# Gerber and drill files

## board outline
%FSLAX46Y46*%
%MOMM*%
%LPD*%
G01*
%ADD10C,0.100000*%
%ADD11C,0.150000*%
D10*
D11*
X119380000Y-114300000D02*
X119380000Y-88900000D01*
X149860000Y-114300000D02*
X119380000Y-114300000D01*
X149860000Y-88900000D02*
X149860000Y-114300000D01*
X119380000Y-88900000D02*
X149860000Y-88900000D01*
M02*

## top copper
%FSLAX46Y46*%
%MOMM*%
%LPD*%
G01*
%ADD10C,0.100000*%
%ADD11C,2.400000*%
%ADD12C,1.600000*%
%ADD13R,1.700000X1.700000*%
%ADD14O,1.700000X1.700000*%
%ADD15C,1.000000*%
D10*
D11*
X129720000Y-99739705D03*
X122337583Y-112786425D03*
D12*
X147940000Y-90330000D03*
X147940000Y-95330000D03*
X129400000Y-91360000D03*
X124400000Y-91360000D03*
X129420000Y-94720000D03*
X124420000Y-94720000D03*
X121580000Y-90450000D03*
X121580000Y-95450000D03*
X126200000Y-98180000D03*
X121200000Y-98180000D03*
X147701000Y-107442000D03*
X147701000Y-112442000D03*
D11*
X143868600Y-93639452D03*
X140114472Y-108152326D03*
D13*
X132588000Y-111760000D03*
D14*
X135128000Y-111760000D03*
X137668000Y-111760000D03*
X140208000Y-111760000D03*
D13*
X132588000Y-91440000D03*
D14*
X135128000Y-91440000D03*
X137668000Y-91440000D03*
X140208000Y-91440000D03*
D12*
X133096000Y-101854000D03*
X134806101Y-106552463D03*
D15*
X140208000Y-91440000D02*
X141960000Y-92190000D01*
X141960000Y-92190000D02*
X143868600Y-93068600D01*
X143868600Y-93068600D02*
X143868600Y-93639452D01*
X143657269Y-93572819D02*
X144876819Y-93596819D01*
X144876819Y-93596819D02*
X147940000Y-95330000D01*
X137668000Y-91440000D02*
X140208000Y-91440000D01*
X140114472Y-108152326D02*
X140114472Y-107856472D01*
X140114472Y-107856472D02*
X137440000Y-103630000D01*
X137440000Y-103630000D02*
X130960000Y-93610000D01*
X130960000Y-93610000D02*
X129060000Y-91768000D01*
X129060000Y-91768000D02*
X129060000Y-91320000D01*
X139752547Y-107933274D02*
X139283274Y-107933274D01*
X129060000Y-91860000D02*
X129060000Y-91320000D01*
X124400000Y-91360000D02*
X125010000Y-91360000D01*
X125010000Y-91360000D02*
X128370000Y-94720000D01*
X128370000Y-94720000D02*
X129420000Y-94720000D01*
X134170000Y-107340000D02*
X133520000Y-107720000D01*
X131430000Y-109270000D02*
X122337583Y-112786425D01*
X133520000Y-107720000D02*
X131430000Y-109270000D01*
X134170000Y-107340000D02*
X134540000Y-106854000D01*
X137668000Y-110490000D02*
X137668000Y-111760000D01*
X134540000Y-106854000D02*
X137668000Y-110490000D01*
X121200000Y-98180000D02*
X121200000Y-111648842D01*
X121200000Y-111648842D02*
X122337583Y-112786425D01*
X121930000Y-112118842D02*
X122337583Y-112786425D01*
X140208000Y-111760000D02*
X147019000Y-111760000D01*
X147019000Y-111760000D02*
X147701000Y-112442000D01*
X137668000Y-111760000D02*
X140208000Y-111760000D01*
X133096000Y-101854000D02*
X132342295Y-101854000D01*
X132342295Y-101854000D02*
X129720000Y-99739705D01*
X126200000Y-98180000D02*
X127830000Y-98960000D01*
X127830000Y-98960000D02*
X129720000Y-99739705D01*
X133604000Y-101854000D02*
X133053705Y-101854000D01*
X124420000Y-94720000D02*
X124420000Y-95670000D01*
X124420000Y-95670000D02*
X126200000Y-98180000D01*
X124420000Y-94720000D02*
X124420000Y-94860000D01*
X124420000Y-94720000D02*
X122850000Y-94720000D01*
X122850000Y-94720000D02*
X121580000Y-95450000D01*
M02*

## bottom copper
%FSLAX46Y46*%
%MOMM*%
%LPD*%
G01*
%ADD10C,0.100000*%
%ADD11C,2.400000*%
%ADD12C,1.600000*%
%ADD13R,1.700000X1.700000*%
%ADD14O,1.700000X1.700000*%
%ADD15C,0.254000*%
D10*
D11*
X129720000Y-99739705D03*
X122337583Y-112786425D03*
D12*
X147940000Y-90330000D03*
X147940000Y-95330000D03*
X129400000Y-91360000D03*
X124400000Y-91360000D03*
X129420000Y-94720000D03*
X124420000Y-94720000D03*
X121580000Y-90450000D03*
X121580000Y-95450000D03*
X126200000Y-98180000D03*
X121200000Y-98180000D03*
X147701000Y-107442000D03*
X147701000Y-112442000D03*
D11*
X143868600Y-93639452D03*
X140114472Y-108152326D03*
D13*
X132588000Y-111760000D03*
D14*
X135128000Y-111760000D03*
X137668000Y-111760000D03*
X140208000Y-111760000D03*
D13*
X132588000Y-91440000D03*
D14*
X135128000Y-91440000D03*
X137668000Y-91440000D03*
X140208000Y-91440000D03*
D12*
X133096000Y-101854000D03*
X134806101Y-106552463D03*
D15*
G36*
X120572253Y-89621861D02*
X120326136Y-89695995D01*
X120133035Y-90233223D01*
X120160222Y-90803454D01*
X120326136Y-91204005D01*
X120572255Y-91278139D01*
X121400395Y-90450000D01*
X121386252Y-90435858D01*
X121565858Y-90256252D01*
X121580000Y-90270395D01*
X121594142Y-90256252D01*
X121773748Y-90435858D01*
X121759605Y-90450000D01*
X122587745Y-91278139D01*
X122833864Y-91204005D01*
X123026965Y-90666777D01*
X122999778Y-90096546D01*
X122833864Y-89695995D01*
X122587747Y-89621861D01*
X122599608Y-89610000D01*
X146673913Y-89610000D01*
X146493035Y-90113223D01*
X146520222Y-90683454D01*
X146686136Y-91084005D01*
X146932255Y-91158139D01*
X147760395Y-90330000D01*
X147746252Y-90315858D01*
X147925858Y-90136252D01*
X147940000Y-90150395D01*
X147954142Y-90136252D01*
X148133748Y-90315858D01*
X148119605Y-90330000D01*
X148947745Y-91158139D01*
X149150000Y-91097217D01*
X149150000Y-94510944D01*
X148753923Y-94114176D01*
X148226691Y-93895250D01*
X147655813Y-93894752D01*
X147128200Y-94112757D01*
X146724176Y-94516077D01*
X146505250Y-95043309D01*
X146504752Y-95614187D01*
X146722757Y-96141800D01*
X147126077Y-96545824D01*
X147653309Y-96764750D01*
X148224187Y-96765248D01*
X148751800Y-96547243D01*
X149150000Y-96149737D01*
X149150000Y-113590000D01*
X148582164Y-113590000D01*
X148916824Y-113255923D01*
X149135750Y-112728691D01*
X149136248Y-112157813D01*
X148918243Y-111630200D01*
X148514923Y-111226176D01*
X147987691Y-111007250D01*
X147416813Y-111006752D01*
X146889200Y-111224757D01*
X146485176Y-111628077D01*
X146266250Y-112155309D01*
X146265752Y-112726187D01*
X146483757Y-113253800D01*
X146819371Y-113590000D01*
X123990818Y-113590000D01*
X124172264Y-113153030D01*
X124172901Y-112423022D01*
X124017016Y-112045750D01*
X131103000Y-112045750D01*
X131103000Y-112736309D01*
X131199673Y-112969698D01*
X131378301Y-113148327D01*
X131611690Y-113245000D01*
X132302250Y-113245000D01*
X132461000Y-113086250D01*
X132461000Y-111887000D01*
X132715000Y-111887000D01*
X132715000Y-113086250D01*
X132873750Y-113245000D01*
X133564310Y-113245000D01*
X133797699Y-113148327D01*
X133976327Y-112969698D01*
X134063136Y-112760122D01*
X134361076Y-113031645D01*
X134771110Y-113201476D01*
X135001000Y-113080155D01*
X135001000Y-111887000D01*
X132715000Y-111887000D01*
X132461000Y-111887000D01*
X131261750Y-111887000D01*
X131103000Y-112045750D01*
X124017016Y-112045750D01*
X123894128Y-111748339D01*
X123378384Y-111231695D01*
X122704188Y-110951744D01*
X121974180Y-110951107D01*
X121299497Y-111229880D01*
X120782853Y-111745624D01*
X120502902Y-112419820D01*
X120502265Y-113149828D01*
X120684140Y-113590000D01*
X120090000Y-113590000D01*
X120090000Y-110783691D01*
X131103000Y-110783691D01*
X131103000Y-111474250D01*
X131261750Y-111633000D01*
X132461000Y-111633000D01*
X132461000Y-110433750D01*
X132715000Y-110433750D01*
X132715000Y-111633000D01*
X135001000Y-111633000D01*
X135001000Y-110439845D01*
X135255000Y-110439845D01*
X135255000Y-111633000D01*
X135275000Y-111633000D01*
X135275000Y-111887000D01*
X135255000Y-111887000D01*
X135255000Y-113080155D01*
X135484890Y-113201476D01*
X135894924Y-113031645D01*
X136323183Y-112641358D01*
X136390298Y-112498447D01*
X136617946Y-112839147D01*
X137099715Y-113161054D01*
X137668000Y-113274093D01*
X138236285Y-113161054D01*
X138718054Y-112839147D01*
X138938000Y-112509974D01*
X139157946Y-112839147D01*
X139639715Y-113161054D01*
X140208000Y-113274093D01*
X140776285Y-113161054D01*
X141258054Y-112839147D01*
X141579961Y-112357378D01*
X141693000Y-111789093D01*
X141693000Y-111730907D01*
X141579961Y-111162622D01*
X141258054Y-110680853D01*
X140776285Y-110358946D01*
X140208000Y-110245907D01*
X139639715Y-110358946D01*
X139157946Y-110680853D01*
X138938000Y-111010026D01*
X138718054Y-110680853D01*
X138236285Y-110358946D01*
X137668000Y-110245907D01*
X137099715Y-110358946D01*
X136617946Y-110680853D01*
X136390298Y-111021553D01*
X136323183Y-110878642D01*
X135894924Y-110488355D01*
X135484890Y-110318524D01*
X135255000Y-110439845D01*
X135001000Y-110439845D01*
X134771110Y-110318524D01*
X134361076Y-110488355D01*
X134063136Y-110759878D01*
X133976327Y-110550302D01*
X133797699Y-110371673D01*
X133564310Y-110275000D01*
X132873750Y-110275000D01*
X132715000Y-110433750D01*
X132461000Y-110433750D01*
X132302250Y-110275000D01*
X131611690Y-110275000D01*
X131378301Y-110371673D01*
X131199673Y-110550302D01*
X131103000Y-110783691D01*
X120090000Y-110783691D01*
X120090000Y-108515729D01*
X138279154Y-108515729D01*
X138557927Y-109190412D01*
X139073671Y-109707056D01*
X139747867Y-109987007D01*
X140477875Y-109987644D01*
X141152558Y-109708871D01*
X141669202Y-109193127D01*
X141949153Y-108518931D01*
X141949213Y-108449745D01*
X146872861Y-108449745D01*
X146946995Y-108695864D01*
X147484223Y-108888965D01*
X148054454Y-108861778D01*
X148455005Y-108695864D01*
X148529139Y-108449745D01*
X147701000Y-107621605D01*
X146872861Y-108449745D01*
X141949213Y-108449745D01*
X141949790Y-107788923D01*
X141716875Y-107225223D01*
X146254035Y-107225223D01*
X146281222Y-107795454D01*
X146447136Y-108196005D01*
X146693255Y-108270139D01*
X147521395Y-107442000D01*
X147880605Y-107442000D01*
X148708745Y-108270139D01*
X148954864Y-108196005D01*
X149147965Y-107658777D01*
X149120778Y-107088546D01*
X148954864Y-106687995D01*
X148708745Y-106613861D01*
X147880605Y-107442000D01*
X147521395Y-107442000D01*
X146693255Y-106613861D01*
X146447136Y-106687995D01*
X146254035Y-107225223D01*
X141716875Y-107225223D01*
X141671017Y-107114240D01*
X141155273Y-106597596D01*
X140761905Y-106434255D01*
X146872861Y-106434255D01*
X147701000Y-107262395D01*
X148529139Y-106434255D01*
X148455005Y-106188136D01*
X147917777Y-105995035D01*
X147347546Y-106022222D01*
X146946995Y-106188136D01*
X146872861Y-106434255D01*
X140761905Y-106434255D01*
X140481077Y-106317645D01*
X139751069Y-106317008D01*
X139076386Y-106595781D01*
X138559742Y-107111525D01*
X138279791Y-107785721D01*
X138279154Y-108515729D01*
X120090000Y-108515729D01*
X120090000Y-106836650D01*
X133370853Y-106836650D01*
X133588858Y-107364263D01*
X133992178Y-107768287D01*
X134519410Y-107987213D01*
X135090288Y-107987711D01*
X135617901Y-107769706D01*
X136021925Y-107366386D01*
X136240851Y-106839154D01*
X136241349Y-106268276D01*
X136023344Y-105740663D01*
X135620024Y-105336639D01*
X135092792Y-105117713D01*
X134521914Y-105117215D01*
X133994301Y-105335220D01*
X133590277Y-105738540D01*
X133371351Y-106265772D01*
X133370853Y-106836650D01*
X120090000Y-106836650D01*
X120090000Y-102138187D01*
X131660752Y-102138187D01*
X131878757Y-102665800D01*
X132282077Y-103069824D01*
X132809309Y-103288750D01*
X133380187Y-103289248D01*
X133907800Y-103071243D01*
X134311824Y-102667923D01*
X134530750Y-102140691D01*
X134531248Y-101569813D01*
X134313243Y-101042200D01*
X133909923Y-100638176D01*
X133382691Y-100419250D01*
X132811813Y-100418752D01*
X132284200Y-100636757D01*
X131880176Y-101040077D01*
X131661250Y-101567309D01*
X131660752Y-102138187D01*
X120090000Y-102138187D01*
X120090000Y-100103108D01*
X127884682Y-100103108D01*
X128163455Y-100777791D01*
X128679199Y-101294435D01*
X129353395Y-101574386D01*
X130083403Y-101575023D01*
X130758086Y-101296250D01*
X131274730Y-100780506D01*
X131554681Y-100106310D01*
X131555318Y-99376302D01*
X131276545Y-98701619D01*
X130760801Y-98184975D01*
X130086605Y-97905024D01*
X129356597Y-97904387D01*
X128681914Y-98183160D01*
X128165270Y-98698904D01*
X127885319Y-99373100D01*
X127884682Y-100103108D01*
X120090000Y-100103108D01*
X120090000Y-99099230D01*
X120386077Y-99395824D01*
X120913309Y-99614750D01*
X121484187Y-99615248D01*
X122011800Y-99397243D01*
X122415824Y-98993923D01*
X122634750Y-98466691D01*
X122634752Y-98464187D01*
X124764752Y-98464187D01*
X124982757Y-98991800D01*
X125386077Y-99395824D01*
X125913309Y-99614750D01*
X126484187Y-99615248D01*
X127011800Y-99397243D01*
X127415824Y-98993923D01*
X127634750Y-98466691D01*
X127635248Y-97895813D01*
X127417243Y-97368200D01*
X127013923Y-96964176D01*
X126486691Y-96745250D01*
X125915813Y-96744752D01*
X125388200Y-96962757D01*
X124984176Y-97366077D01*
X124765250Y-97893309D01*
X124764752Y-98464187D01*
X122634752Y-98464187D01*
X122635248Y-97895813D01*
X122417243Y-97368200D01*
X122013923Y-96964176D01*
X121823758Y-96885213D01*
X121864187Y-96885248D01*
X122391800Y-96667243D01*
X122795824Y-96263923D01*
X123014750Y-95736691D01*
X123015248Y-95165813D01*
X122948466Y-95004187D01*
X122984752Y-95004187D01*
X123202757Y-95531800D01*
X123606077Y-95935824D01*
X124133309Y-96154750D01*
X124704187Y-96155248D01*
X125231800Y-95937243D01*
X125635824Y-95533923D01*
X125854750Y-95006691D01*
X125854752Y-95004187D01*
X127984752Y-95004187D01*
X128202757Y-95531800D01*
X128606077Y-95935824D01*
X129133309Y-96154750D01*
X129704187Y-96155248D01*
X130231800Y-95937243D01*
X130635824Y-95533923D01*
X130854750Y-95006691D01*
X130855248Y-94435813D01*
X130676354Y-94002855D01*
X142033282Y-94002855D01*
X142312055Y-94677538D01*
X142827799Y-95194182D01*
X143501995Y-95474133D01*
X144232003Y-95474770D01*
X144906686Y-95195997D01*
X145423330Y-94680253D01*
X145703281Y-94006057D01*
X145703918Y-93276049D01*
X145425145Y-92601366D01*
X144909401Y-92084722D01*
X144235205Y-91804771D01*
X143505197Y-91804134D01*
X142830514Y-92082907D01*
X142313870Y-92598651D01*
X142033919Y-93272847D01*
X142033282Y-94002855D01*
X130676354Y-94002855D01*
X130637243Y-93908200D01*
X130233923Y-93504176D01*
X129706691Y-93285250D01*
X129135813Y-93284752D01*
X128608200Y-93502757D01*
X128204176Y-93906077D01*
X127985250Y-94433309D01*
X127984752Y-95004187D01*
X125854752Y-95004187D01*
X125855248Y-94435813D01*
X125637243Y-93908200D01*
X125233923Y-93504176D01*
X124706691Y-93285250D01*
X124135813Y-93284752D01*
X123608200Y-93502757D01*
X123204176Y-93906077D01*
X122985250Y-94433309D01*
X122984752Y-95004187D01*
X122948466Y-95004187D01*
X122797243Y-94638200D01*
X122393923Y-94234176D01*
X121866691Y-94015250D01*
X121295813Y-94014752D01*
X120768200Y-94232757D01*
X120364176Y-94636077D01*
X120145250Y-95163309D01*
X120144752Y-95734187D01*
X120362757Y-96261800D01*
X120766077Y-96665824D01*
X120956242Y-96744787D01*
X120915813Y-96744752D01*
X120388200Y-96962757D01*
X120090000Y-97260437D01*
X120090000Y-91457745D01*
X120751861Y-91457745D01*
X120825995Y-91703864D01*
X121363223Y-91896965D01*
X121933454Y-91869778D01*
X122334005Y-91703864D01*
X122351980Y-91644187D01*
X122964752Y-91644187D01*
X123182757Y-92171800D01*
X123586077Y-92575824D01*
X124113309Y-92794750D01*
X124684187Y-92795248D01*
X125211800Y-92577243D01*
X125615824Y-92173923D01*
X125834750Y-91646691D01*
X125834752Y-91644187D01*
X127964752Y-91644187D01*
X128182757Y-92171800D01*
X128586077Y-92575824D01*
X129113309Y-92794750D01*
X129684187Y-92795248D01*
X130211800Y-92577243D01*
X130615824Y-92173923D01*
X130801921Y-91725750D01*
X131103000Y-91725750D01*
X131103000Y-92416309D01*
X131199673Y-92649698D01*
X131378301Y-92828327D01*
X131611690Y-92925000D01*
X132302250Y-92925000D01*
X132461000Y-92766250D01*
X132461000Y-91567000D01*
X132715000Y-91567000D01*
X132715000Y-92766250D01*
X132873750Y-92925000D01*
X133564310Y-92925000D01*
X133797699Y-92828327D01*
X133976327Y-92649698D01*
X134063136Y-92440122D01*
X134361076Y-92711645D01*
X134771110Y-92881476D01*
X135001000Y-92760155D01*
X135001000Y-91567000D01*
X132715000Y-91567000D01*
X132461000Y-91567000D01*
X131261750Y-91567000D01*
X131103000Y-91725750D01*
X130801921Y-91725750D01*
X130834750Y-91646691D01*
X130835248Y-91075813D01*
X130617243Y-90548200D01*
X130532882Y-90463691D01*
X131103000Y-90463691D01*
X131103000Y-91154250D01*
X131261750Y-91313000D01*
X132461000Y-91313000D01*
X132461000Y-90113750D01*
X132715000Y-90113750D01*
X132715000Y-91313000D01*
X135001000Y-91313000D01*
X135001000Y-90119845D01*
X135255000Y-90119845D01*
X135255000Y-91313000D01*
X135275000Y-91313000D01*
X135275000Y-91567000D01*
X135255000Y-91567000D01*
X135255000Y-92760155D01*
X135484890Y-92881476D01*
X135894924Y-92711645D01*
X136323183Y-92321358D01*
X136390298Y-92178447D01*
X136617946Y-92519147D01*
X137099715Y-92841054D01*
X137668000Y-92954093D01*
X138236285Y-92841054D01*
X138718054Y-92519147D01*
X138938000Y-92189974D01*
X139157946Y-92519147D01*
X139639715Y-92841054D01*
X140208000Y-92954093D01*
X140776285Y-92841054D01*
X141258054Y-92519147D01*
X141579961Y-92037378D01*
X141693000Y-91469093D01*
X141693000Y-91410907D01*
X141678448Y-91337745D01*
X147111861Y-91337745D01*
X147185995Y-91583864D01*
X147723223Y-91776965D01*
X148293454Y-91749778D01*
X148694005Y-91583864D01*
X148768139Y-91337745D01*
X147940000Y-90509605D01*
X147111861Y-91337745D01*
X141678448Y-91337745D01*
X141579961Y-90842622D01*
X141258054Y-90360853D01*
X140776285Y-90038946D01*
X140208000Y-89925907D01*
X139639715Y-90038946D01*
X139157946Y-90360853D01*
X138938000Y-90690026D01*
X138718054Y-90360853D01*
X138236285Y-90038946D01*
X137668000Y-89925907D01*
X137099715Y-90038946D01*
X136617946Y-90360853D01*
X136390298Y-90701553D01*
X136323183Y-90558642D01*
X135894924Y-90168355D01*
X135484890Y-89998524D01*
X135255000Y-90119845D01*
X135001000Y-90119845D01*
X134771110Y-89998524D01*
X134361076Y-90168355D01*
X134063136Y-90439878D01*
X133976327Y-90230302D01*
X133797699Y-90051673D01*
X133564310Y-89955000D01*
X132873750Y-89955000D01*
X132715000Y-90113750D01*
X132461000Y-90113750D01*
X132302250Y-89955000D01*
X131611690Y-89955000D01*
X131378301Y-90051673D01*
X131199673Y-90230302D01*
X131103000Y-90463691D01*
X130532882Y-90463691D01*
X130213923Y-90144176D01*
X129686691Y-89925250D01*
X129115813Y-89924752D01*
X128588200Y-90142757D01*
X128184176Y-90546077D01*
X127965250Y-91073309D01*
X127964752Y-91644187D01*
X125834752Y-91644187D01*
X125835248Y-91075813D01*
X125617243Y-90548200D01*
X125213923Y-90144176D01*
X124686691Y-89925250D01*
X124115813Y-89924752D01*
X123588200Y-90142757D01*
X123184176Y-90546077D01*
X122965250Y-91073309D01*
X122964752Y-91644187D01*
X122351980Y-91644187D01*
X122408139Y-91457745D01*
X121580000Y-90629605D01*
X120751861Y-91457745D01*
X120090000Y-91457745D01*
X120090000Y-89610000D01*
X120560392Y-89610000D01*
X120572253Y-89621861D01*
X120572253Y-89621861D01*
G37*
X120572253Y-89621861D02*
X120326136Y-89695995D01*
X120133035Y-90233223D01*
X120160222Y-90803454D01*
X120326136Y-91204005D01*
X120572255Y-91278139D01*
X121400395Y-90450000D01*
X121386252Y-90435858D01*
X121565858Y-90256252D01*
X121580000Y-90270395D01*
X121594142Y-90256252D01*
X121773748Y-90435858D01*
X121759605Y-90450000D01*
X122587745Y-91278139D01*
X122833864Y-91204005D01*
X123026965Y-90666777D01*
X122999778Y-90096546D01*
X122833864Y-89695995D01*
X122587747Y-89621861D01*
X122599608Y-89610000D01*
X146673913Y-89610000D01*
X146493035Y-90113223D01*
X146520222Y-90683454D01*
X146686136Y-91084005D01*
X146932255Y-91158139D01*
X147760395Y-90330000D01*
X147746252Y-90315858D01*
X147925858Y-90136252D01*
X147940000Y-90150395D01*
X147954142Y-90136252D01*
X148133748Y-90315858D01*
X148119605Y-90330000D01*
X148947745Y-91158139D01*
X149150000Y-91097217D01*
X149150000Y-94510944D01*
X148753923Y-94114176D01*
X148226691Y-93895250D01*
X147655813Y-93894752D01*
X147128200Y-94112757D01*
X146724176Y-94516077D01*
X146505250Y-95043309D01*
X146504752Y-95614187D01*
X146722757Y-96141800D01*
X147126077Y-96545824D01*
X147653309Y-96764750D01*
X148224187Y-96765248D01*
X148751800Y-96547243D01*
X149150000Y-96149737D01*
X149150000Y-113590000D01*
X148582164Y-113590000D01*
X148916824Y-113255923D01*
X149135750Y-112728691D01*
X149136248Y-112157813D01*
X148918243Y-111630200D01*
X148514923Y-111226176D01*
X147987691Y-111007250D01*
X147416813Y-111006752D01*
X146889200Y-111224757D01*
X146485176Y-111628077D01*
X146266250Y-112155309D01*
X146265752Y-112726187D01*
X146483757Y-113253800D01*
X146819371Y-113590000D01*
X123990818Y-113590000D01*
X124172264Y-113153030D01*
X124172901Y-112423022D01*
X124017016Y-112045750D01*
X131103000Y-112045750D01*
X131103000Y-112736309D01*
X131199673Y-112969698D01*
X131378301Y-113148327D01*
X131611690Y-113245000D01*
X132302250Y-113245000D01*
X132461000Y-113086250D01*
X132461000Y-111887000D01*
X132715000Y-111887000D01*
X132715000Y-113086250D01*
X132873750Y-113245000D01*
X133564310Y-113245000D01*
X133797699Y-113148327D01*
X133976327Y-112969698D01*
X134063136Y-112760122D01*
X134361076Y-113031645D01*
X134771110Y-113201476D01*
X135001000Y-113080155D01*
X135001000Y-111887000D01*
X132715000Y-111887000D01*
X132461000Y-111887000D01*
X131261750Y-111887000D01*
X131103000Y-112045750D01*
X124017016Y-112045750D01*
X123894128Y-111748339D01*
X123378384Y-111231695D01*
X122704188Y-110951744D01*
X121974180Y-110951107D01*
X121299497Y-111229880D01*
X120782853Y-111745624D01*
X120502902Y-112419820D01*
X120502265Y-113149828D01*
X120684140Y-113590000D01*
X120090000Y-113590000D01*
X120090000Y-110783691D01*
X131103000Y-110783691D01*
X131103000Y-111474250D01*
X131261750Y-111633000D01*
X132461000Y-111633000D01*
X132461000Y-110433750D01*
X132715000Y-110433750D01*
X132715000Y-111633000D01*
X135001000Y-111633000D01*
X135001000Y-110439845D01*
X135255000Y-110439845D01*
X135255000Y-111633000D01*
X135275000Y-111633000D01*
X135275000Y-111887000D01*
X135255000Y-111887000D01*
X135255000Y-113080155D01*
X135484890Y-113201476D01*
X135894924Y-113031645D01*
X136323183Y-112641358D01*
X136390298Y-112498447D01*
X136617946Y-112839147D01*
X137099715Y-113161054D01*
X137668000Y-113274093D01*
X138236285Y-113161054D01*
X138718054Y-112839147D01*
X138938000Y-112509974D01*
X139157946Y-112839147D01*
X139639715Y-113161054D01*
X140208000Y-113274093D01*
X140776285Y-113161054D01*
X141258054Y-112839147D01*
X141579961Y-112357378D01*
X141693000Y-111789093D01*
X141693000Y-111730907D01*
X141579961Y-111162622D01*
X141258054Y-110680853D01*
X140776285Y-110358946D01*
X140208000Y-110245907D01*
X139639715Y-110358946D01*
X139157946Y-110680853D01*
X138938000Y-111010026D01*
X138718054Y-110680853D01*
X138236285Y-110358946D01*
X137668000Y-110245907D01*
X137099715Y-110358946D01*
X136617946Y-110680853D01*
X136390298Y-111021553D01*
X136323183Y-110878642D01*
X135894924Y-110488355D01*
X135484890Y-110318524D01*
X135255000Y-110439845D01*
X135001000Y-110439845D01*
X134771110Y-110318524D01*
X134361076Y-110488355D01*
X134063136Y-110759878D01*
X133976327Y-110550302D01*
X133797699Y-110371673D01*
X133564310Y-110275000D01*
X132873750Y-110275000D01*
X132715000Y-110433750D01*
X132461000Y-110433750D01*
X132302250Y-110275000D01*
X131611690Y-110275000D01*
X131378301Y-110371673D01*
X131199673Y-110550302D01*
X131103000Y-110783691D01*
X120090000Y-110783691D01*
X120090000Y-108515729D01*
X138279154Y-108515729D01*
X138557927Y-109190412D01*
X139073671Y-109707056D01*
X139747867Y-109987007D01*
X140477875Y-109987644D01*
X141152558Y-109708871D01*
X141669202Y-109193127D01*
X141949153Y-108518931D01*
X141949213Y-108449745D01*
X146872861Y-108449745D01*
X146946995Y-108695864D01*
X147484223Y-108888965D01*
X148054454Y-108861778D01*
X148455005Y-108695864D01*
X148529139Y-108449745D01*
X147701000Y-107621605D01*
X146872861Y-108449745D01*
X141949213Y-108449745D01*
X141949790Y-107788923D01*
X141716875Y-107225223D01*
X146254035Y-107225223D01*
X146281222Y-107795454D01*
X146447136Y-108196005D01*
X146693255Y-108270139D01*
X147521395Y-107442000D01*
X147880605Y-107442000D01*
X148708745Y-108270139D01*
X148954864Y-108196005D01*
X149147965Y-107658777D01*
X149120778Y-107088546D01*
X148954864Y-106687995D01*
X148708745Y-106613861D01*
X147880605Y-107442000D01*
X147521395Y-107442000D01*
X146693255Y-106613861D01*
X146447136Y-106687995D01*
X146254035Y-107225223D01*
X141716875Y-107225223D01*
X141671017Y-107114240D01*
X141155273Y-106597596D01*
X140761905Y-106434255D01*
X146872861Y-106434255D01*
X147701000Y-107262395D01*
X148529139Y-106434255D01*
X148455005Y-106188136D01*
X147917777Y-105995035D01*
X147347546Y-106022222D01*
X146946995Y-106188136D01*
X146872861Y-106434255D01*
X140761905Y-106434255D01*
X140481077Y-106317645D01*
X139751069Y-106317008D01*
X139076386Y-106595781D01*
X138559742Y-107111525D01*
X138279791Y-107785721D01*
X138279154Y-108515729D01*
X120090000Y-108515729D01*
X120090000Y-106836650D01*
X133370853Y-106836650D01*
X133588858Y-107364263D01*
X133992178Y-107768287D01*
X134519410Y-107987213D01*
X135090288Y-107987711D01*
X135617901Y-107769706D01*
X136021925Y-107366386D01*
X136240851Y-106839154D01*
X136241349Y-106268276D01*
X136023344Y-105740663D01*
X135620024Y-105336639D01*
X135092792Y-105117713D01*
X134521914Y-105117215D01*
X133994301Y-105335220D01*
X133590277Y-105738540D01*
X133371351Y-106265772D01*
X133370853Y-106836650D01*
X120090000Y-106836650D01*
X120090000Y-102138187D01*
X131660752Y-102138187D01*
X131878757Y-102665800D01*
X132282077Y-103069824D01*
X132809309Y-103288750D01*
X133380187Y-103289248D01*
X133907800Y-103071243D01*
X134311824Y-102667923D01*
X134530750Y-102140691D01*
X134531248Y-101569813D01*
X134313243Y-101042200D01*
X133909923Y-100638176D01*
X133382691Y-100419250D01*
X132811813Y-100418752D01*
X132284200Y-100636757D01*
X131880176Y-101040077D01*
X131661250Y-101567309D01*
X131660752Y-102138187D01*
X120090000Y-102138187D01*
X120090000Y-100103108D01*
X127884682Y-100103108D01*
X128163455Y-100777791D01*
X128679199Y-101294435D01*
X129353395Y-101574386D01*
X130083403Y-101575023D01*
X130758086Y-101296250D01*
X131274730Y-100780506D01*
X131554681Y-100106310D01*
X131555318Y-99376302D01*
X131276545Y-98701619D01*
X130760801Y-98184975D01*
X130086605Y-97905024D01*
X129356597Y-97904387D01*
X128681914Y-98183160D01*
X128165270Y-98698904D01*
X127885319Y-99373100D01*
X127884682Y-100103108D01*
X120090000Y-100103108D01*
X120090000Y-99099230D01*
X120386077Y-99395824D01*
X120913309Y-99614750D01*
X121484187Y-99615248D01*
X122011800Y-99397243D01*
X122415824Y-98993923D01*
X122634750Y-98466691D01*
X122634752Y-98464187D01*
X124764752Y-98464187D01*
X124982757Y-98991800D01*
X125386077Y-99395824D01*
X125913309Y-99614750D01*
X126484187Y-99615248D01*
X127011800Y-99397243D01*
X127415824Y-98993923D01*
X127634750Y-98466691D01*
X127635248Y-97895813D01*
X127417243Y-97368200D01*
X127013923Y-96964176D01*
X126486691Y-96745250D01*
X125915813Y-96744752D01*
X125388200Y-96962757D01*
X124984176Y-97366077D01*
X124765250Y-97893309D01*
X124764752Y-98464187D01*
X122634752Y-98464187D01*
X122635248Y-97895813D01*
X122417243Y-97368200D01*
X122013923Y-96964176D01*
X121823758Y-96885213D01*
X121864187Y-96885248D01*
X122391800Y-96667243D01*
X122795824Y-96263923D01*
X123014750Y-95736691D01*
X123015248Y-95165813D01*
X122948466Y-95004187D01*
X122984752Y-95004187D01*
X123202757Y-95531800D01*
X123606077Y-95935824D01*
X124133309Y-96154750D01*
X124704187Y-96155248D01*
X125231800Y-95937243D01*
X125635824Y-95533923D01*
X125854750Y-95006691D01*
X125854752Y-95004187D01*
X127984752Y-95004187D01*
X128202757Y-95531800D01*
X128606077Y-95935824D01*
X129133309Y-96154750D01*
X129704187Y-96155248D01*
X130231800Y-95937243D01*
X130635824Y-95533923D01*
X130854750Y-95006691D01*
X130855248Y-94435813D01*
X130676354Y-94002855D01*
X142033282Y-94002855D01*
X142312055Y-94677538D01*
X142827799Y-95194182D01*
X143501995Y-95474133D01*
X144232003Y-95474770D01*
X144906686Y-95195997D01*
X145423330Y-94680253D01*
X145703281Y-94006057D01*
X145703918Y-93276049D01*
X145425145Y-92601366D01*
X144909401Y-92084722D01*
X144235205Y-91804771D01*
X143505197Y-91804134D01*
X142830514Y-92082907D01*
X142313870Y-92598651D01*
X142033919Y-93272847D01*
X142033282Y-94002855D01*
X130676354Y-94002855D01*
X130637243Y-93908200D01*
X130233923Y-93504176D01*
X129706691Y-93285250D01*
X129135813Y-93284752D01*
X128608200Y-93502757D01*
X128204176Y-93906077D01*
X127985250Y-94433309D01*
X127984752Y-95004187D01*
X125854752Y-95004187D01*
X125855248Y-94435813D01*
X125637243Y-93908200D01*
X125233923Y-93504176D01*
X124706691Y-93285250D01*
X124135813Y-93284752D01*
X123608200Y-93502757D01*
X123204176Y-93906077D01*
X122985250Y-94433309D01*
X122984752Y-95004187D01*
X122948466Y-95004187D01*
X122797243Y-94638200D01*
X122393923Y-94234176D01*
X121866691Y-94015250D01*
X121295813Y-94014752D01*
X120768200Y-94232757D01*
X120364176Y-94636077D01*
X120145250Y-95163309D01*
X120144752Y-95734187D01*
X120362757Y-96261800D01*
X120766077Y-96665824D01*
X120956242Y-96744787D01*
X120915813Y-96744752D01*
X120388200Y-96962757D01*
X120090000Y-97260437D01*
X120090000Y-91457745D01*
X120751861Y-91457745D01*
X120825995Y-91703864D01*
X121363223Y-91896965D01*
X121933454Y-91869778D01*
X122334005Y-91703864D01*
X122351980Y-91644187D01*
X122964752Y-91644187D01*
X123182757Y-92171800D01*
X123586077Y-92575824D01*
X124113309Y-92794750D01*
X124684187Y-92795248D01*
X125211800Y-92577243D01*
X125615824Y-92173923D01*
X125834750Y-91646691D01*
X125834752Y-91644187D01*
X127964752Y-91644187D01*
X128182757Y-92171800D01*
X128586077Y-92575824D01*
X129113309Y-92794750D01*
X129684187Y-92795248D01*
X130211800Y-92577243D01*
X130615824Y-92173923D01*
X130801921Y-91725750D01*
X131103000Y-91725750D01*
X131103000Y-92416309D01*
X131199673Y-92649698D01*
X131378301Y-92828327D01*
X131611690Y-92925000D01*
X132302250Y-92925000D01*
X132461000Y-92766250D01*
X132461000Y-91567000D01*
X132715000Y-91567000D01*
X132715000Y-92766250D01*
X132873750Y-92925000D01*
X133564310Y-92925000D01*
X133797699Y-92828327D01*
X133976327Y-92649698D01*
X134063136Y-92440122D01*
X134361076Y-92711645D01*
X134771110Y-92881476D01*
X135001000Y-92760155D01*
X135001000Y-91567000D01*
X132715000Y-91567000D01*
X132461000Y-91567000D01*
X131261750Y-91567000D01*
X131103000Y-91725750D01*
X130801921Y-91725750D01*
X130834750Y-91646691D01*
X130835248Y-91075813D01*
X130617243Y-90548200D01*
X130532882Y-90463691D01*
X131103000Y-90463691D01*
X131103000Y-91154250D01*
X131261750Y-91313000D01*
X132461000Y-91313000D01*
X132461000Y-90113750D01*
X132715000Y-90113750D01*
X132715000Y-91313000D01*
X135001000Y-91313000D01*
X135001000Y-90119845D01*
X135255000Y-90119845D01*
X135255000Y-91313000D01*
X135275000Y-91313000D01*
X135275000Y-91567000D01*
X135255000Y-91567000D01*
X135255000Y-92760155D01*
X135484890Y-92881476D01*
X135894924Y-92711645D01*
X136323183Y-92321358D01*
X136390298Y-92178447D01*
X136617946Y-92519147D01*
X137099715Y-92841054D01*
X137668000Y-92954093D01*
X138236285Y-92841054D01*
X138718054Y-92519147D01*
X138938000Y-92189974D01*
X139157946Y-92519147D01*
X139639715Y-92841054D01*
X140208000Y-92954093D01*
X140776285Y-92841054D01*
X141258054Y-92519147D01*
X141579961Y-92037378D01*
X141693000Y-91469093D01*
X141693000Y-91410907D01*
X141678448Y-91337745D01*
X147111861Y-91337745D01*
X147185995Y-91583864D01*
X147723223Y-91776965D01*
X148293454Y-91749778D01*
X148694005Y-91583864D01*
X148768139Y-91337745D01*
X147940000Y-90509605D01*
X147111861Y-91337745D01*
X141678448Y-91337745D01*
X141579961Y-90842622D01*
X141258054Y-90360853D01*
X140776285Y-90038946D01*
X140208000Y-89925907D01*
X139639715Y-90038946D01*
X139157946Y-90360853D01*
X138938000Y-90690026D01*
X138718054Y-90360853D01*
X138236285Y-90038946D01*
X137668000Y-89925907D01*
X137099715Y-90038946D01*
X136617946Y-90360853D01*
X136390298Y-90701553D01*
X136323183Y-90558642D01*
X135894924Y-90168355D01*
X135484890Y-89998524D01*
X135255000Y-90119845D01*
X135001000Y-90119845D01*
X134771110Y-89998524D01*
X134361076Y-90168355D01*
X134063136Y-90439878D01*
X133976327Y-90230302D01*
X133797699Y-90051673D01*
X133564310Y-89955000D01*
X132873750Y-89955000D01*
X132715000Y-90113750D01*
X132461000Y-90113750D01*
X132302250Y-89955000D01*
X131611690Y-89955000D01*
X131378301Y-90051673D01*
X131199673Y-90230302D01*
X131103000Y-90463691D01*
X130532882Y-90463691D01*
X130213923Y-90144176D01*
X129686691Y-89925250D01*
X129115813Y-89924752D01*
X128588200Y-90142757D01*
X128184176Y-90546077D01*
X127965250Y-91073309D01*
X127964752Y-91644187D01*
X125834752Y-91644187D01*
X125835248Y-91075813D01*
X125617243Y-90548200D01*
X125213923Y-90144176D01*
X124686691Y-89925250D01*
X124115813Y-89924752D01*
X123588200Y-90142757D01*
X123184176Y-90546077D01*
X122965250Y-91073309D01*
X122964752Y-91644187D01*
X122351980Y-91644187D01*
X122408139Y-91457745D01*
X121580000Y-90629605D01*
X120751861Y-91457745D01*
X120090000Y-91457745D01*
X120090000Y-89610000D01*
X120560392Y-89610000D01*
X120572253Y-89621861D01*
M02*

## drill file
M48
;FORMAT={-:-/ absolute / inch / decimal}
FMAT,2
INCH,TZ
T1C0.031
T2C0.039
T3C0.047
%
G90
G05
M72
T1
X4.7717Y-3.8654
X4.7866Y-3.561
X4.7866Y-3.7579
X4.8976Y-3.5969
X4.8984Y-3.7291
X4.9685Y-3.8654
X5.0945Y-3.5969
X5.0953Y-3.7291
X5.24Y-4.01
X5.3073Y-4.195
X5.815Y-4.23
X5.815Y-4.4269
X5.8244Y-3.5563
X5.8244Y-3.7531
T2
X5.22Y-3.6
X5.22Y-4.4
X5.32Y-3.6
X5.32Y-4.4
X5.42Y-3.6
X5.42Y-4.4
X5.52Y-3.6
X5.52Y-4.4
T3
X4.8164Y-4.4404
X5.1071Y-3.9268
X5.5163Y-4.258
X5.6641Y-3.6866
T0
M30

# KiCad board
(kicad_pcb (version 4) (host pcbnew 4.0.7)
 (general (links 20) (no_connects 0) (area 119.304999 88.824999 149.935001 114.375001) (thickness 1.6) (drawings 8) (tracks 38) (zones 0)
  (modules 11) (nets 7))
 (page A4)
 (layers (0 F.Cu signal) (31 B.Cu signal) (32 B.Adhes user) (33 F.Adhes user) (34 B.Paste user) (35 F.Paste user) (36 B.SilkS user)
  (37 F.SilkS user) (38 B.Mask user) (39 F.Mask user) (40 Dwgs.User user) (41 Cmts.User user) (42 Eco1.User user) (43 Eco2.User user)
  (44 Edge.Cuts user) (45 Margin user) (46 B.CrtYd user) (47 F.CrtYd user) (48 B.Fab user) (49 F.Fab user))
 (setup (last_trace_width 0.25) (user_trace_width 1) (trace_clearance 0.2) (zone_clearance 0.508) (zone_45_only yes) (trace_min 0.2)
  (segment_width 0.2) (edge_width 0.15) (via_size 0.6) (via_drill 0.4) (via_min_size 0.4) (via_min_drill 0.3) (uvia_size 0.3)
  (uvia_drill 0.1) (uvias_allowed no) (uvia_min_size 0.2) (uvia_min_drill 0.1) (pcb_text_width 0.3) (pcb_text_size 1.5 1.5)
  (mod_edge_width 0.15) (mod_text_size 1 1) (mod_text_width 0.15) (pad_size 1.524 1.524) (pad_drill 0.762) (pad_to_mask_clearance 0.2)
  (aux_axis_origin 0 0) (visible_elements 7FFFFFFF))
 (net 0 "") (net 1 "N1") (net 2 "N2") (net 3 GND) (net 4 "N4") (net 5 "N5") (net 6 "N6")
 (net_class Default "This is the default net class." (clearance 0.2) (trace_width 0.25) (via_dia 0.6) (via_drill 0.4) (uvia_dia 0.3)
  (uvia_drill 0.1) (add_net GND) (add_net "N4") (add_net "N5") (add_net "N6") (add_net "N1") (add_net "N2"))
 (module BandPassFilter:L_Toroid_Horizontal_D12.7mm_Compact (layer F.Cu) (at 130.99 97.54 240)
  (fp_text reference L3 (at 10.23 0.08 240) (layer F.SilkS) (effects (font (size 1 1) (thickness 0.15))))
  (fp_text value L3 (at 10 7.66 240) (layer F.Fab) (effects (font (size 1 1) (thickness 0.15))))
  (pad 1 thru_hole circle (at 2.54 0 240) (size 2.4 2.4) (drill 1.2) (layers *.Cu *.Mask) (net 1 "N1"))
  (pad 2 thru_hole circle (at 17.53 -0.13 240) (size 2.4 2.4) (drill 1.2) (layers *.Cu *.Mask) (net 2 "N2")))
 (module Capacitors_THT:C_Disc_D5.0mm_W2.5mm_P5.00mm (layer F.Cu) (at 147.94 90.33 270)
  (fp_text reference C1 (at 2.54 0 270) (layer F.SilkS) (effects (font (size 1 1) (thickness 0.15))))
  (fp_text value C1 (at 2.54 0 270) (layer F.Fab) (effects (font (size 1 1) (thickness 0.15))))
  (pad 1 thru_hole circle (at 0 0 270) (size 1.6 1.6) (drill 0.8) (layers *.Cu *.Mask) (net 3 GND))
  (pad 2 thru_hole circle (at 5 0 270) (size 1.6 1.6) (drill 0.8) (layers *.Cu *.Mask) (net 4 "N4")))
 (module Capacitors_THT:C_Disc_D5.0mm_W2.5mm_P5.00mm (layer F.Cu) (at 129.4 91.36 180)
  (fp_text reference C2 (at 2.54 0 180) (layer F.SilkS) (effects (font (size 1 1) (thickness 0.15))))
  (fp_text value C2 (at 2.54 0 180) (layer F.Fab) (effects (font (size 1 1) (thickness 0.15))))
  (pad 1 thru_hole circle (at 0 0 180) (size 1.6 1.6) (drill 0.8) (layers *.Cu *.Mask) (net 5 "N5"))
  (pad 2 thru_hole circle (at 5 0 180) (size 1.6 1.6) (drill 0.8) (layers *.Cu *.Mask) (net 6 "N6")))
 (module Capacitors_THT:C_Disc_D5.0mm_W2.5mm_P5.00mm (layer F.Cu) (at 129.42 94.72 180)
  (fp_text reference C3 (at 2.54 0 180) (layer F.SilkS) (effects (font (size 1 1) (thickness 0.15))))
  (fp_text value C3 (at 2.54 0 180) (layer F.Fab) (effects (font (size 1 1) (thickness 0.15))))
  (pad 1 thru_hole circle (at 0 0 180) (size 1.6 1.6) (drill 0.8) (layers *.Cu *.Mask) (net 6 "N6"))
  (pad 2 thru_hole circle (at 5 0 180) (size 1.6 1.6) (drill 0.8) (layers *.Cu *.Mask) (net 1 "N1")))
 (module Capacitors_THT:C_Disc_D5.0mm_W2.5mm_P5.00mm (layer F.Cu) (at 121.58 90.45 270)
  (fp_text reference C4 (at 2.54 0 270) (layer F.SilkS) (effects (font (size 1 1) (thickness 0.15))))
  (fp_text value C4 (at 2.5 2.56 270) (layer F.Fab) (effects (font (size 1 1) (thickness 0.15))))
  (pad 1 thru_hole circle (at 0 0 270) (size 1.6 1.6) (drill 0.8) (layers *.Cu *.Mask) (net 3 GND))
  (pad 2 thru_hole circle (at 5 0 270) (size 1.6 1.6) (drill 0.8) (layers *.Cu *.Mask) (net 1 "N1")))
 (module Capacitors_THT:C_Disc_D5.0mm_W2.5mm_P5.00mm (layer F.Cu) (at 126.2 98.18 180)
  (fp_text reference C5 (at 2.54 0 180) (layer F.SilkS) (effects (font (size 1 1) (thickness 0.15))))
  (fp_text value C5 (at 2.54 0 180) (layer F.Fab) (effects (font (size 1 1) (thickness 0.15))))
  (pad 1 thru_hole circle (at 0 0 180) (size 1.6 1.6) (drill 0.8) (layers *.Cu *.Mask) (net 1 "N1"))
  (pad 2 thru_hole circle (at 5 0 180) (size 1.6 1.6) (drill 0.8) (layers *.Cu *.Mask) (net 2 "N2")))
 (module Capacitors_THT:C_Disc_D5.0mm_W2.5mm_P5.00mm (layer F.Cu) (at 147.701 107.442 270)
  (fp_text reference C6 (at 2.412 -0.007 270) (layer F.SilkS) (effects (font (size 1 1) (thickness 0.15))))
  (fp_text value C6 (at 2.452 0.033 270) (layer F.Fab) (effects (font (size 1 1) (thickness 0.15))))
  (pad 1 thru_hole circle (at 0 0 270) (size 1.6 1.6) (drill 0.8) (layers *.Cu *.Mask) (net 3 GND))
  (pad 2 thru_hole circle (at 5 0 270) (size 1.6 1.6) (drill 0.8) (layers *.Cu *.Mask) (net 2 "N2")))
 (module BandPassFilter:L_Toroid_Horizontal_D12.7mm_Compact (layer F.Cu) (at 144.526 91.186 255)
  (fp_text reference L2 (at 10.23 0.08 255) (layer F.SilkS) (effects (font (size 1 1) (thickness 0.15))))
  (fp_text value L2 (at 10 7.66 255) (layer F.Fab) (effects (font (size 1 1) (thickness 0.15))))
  (pad 1 thru_hole circle (at 2.54 0 255) (size 2.4 2.4) (drill 1.2) (layers *.Cu *.Mask) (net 4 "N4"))
  (pad 2 thru_hole circle (at 17.53 -0.13 255) (size 2.4 2.4) (drill 1.2) (layers *.Cu *.Mask) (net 5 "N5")))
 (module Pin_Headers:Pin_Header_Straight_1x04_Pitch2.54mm (layer F.Cu) (at 132.588 111.76 90)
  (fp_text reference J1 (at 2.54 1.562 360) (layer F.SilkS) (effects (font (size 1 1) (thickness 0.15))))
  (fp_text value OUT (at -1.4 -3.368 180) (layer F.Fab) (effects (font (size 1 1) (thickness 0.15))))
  (pad 1 thru_hole rect (at 0 0 90) (size 1.7 1.7) (drill 1) (layers *.Cu *.Mask) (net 3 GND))
  (pad 2 thru_hole oval (at 0 2.54 90) (size 1.7 1.7) (drill 1) (layers *.Cu *.Mask) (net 3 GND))
  (pad 3 thru_hole oval (at 0 5.08 90) (size 1.7 1.7) (drill 1) (layers *.Cu *.Mask) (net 2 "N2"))
  (pad 4 thru_hole oval (at 0 7.62 90) (size 1.7 1.7) (drill 1) (layers *.Cu *.Mask) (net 2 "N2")))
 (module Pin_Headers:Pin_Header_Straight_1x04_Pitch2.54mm (layer F.Cu) (at 132.588 91.44 90)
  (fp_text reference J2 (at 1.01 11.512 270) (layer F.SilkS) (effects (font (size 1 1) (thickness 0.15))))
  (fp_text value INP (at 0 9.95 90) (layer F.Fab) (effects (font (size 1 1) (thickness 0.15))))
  (pad 1 thru_hole rect (at 0 0 90) (size 1.7 1.7) (drill 1) (layers *.Cu *.Mask) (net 3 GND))
  (pad 2 thru_hole oval (at 0 2.54 90) (size 1.7 1.7) (drill 1) (layers *.Cu *.Mask) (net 3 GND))
  (pad 3 thru_hole oval (at 0 5.08 90) (size 1.7 1.7) (drill 1) (layers *.Cu *.Mask) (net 4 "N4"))
  (pad 4 thru_hole oval (at 0 7.62 90) (size 1.7 1.7) (drill 1) (layers *.Cu *.Mask) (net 4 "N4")))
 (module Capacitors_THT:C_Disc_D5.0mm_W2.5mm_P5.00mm (layer F.Cu) (at 133.096 101.854 290)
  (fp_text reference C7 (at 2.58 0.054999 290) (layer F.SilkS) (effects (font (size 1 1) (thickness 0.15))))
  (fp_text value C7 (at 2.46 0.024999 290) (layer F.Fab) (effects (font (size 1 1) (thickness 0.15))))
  (pad 1 thru_hole circle (at 0 0 290) (size 1.6 1.6) (drill 0.8) (layers *.Cu *.Mask) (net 1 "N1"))
  (pad 2 thru_hole circle (at 5 0 290) (size 1.6 1.6) (drill 0.8) (layers *.Cu *.Mask) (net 2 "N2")))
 (gr_line (start 119.38 114.3) (end 119.38 88.9) (angle 90) (layer Edge.Cuts) (width 0.15))
 (gr_line (start 149.86 114.3) (end 119.38 114.3) (angle 90) (layer Edge.Cuts) (width 0.15))
 (gr_line (start 149.86 88.9) (end 149.86 114.3) (angle 90) (layer Edge.Cuts) (width 0.15))
 (gr_line (start 119.38 88.9) (end 149.86 88.9) (angle 90) (layer Edge.Cuts) (width 0.15))
 (segment (start 140.208 91.44) (end 141.96 92.19) (width 1) (layer F.Cu) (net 4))
 (segment (start 141.96 92.19) (end 143.8686 93.0686) (width 1) (layer F.Cu) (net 4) (status 20))
 (segment (start 143.8686 93.0686) (end 143.8686 93.639452) (width 1) (layer F.Cu) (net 4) (status 30))
 (segment (start 143.657269 93.572819) (end 144.876819 93.596819) (width 1) (layer F.Cu) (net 4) (status 30))
 (segment (start 144.876819 93.596819) (end 147.94 95.33) (width 1) (layer F.Cu) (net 4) (status 10))
 (segment (start 137.668 91.44) (end 140.208 91.44) (width 1) (layer F.Cu) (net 4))
 (segment (start 140.114472 108.152326) (end 140.114472 107.856472) (width 1) (layer F.Cu) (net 5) (status 30))
 (segment (start 140.114472 107.856472) (end 137.44 103.63) (width 1) (layer F.Cu) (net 5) (status 10))
 (segment (start 137.44 103.63) (end 130.96 93.61) (width 1) (layer F.Cu) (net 5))
 (segment (start 130.96 93.61) (end 129.06 91.768) (width 1) (layer F.Cu) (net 5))
 (segment (start 129.06 91.768) (end 129.06 91.32) (width 1) (layer F.Cu) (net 5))
 (segment (start 139.752547 107.933274) (end 139.283274 107.933274) (width 1) (layer F.Cu) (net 5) (status 30))
 (segment (start 129.06 91.86) (end 129.06 91.32) (width 1) (layer F.Cu) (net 5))
 (segment (start 124.4 91.36) (end 125.01 91.36) (width 1) (layer F.Cu) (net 6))
 (segment (start 125.01 91.36) (end 128.37 94.72) (width 1) (layer F.Cu) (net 6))
 (segment (start 128.37 94.72) (end 129.42 94.72) (width 1) (layer F.Cu) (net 6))
 (segment (start 134.17 107.34) (end 133.52 107.72) (width 1) (layer F.Cu) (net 2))
 (segment (start 131.43 109.27) (end 122.337583 112.786425) (width 1) (layer F.Cu) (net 2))
 (segment (start 133.52 107.72) (end 131.43 109.27) (width 1) (layer F.Cu) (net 2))
 (segment (start 134.17 107.34) (end 134.54 106.854) (width 1) (layer F.Cu) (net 2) (status 20))
 (segment (start 137.668 110.49) (end 137.668 111.76) (width 1) (layer F.Cu) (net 2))
 (segment (start 134.54 106.854) (end 137.668 110.49) (width 1) (layer F.Cu) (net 2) (status 10))
 (segment (start 121.2 98.18) (end 121.2 111.648842) (width 1) (layer F.Cu) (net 2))
 (segment (start 121.2 111.648842) (end 122.337583 112.786425) (width 1) (layer F.Cu) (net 2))
 (segment (start 121.93 112.118842) (end 122.337583 112.786425) (width 1) (layer F.Cu) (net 2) (status 30))
 (segment (start 140.208 111.76) (end 147.019 111.76) (width 1) (layer F.Cu) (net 2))
 (segment (start 147.019 111.76) (end 147.701 112.442) (width 1) (layer F.Cu) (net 2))
 (segment (start 137.668 111.76) (end 140.208 111.76) (width 1) (layer F.Cu) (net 2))
 (segment (start 133.096 101.854) (end 132.342295 101.854) (width 1) (layer F.Cu) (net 1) (status 30))
 (segment (start 132.342295 101.854) (end 129.72 99.739705) (width 1) (layer F.Cu) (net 1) (status 10))
 (segment (start 126.2 98.18) (end 127.83 98.96) (width 1) (layer F.Cu) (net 1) (status 10))
 (segment (start 127.83 98.96) (end 129.72 99.739705) (width 1) (layer F.Cu) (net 1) (status 20))
 (segment (start 133.604 101.854) (end 133.053705 101.854) (width 1) (layer F.Cu) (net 1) (status 30))
 (segment (start 124.42 94.72) (end 124.42 95.67) (width 1) (layer F.Cu) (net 1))
 (segment (start 124.42 95.67) (end 126.2 98.18) (width 1) (layer F.Cu) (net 1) (status 20))
 (segment (start 124.42 94.72) (end 124.42 94.86) (width 1) (layer F.Cu) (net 1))
 (segment (start 124.42 94.72) (end 122.85 94.72) (width 1) (layer F.Cu) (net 1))
 (segment (start 122.85 94.72) (end 121.58 95.45) (width 1) (layer F.Cu) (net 1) (status 20))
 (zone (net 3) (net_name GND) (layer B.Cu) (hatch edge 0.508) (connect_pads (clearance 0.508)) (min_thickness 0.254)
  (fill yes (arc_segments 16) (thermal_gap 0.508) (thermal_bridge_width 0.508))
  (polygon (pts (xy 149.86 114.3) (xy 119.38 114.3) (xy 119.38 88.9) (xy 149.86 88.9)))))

